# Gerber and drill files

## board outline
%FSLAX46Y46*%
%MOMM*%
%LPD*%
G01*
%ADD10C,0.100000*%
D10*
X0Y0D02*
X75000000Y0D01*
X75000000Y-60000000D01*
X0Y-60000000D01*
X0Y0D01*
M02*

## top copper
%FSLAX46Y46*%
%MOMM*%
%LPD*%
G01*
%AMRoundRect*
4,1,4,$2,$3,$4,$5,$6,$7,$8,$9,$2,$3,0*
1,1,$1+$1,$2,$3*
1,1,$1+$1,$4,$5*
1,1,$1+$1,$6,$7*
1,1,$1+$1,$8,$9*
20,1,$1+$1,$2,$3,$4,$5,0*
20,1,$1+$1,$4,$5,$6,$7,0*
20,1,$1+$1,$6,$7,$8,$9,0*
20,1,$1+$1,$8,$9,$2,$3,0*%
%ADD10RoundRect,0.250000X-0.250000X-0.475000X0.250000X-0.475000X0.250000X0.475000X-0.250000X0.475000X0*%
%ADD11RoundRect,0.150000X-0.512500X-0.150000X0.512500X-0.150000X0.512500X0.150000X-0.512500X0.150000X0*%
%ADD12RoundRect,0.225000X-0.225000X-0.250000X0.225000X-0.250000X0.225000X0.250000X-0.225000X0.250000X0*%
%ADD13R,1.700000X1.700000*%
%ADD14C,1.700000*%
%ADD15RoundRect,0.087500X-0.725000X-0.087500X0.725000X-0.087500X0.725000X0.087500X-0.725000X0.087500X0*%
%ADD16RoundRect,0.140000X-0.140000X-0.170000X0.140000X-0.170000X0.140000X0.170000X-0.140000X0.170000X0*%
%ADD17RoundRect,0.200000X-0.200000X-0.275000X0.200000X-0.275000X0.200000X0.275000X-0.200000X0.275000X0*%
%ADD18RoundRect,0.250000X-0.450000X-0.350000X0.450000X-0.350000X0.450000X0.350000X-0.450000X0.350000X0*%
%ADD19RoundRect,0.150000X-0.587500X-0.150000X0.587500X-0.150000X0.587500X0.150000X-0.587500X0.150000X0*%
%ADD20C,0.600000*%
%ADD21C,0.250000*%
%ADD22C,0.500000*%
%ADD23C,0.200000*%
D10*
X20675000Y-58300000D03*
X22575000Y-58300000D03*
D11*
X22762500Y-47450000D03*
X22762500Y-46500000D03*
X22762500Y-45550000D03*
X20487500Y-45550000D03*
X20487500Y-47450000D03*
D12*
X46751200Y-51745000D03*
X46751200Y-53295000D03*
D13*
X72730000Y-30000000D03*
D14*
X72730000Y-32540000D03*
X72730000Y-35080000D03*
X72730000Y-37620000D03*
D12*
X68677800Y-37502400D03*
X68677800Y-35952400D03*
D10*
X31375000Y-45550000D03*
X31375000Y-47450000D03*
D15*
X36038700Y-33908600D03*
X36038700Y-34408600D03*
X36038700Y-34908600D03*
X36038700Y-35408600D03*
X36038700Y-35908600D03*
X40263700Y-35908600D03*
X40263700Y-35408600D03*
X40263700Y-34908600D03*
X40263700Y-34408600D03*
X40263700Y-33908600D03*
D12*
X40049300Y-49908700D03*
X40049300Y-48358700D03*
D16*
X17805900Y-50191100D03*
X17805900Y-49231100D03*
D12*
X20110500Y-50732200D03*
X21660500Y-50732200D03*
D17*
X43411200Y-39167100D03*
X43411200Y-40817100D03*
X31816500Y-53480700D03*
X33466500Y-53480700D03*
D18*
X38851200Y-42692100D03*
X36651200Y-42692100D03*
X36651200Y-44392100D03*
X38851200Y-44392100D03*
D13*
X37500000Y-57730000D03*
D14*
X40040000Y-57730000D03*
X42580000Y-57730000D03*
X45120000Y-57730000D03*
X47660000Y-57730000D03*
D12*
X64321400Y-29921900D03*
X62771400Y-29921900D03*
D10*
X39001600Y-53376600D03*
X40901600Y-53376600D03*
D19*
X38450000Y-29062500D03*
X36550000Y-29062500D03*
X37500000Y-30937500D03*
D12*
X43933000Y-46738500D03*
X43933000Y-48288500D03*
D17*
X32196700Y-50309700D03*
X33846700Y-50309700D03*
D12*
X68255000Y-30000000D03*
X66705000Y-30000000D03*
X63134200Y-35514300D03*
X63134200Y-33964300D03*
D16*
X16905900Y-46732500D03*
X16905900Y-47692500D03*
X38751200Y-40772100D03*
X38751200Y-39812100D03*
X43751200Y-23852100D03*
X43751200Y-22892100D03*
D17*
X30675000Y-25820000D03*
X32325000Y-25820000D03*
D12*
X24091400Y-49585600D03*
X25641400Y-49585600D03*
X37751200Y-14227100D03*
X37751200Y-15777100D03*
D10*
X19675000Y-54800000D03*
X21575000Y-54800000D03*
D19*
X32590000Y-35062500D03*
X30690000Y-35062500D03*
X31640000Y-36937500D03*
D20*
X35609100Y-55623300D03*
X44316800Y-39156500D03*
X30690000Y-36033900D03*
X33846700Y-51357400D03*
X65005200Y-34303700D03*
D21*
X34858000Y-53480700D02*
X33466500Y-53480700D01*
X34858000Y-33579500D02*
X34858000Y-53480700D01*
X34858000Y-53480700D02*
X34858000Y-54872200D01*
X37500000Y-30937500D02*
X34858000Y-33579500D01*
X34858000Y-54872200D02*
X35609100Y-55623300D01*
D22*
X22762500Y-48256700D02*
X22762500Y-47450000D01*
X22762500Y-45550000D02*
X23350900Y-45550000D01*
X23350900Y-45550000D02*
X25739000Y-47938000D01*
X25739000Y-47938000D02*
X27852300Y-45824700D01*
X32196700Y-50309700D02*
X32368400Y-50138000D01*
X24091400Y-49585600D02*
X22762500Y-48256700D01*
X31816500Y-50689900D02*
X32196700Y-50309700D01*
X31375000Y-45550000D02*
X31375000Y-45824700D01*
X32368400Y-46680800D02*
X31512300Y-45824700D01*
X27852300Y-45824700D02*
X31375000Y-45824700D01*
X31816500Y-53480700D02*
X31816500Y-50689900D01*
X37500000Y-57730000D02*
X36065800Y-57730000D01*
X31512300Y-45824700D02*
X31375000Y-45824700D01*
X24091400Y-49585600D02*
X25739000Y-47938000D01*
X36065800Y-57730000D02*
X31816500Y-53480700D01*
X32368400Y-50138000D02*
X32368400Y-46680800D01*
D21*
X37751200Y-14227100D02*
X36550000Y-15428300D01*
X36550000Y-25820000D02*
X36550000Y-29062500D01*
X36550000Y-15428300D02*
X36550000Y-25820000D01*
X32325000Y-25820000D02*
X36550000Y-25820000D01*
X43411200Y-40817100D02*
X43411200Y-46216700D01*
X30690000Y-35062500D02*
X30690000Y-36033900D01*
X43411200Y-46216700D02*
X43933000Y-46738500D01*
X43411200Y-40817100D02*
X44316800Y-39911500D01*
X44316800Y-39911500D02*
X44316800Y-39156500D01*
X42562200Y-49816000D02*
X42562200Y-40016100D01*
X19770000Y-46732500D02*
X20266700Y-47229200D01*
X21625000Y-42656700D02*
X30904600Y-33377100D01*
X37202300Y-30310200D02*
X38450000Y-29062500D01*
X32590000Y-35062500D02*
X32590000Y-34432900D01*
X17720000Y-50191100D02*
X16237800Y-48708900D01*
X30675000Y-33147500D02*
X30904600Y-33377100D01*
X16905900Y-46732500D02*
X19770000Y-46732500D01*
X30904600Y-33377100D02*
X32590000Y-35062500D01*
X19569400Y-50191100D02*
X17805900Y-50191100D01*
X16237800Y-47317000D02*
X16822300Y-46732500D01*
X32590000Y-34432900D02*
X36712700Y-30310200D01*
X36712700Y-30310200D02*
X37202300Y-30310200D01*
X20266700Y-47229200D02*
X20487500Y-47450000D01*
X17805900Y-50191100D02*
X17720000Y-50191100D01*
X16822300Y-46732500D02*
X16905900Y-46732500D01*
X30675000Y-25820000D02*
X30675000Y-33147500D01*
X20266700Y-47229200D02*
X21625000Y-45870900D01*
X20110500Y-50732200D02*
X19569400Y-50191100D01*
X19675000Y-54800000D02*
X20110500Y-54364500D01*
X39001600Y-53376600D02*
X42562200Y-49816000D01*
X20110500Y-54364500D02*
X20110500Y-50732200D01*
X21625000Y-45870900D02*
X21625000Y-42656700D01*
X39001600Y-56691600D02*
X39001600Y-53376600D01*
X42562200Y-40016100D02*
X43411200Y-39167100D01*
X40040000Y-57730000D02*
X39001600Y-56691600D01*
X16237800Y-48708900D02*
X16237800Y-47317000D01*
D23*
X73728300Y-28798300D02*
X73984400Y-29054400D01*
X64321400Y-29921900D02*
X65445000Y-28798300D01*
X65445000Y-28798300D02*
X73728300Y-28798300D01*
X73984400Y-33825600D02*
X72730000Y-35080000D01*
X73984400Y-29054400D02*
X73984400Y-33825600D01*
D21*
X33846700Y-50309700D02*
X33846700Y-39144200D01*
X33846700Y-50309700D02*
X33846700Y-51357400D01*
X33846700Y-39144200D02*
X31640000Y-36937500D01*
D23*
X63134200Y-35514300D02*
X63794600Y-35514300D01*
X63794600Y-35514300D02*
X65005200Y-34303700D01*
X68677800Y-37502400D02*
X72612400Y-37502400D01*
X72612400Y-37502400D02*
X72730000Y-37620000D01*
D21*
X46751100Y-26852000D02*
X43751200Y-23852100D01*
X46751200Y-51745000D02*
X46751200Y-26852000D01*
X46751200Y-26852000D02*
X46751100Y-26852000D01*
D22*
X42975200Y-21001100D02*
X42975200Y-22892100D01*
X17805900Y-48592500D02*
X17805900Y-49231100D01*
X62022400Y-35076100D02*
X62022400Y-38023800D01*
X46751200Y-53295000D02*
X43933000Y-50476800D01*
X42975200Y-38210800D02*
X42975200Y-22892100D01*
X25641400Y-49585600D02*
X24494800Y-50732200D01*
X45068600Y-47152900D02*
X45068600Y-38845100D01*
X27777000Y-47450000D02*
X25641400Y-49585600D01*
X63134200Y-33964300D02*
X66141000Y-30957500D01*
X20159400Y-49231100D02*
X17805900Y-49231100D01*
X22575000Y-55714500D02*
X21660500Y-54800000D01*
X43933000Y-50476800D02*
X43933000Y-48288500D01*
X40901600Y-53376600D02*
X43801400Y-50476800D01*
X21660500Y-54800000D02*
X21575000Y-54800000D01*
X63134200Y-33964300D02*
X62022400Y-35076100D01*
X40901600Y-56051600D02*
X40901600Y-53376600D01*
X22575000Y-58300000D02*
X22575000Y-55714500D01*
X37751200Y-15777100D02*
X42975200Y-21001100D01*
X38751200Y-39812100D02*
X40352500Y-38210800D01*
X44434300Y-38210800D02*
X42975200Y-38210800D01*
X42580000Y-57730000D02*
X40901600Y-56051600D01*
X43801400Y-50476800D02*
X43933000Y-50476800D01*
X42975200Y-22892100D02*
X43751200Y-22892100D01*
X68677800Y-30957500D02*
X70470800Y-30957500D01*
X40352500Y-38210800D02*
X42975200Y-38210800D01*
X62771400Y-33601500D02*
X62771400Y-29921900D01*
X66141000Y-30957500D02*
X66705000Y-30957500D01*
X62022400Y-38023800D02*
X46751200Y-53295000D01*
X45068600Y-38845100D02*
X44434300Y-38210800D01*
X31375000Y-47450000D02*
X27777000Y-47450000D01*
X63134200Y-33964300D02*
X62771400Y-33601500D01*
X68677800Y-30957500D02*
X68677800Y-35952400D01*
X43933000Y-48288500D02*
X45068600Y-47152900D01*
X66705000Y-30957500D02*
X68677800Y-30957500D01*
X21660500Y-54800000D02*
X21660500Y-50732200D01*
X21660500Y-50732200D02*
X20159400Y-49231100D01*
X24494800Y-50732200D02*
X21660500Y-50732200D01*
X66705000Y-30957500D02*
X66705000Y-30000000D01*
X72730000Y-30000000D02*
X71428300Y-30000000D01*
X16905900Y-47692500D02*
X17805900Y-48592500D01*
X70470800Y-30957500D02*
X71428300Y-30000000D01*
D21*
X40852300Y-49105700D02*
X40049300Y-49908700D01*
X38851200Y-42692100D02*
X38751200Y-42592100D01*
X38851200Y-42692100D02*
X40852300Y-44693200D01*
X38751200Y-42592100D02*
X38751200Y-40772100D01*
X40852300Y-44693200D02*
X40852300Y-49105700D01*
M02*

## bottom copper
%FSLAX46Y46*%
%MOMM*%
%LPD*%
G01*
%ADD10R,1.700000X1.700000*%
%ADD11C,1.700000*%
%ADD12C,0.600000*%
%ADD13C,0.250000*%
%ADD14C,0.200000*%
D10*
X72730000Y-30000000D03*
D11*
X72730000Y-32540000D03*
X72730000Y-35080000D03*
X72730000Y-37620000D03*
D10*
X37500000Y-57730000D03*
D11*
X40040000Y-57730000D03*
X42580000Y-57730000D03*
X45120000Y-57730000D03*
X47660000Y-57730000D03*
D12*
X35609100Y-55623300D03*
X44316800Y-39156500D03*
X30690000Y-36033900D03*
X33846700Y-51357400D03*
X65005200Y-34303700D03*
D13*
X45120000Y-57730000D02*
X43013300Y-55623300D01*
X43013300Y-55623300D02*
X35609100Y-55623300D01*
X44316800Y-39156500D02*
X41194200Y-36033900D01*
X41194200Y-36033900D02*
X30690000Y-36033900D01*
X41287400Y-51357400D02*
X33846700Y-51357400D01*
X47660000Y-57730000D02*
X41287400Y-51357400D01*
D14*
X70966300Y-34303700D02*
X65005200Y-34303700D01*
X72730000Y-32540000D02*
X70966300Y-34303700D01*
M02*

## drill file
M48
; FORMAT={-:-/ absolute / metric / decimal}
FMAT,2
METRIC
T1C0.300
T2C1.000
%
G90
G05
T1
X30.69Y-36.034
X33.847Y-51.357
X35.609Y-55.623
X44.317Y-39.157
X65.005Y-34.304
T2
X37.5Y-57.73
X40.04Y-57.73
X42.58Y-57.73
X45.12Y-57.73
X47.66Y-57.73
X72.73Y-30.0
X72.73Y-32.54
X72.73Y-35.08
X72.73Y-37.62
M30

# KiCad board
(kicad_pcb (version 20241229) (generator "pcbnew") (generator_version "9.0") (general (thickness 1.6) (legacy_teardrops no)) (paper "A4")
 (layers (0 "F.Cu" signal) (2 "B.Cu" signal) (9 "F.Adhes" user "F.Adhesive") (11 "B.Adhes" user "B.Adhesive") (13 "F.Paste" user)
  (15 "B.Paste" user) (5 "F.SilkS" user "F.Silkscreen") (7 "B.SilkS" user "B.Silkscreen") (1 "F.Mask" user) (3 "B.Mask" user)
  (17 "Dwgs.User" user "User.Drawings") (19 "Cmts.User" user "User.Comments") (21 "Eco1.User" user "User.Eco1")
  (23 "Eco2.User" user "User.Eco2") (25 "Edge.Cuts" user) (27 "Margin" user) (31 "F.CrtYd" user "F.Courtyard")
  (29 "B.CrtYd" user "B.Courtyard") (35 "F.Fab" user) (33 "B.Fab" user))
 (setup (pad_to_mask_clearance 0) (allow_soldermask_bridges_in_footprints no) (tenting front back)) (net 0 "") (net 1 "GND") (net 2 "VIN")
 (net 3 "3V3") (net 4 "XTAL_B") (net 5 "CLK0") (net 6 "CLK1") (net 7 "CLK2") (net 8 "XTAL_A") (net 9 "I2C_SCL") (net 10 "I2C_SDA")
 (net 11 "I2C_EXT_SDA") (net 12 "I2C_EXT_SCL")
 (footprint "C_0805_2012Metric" (layer "F.Cu") (at 21.625 58.3)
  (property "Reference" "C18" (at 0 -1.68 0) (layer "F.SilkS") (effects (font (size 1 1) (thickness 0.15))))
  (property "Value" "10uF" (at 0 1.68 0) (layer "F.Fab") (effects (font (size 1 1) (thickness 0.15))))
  (pad "1" smd roundrect (at -0.95 0) (size 1 1.45) (layers "F.Cu" "F.Mask" "F.Paste") (roundrect_rratio 0.25))
  (pad "2" smd roundrect (at 0.95 0) (size 1 1.45) (layers "F.Cu" "F.Mask" "F.Paste") (roundrect_rratio 0.25) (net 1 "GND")))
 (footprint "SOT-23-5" (layer "F.Cu") (at 21.625 46.5 180)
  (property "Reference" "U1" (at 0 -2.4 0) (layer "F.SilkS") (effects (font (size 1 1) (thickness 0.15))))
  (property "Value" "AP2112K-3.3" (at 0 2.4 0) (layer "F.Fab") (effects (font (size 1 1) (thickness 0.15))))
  (pad "1" smd roundrect (at -1.1375 -0.95) (size 1.325 0.6) (layers "F.Cu" "F.Mask" "F.Paste") (roundrect_rratio 0.25) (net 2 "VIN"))
  (pad "2" smd roundrect (at -1.1375 0) (size 1.325 0.6) (layers "F.Cu" "F.Mask" "F.Paste") (roundrect_rratio 0.25) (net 1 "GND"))
  (pad "3" smd roundrect (at -1.1375 0.95) (size 1.325 0.6) (layers "F.Cu" "F.Mask" "F.Paste") (roundrect_rratio 0.25) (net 2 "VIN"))
  (pad "4" smd roundrect (at 1.1375 0.95) (size 1.325 0.6) (layers "F.Cu" "F.Mask" "F.Paste") (roundrect_rratio 0.25))
  (pad "5" smd roundrect (at 1.1375 -0.95) (size 1.325 0.6) (layers "F.Cu" "F.Mask" "F.Paste") (roundrect_rratio 0.25) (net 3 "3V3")))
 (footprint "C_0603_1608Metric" (layer "F.Cu") (at 46.7512 52.52 -90)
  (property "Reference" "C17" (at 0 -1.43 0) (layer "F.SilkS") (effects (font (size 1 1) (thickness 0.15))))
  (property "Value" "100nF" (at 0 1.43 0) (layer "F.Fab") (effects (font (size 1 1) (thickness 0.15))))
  (pad "1" smd roundrect (at -0.775 0) (size 0.9 0.95) (layers "F.Cu" "F.Mask" "F.Paste") (roundrect_rratio 0.25) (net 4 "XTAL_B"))
  (pad "2" smd roundrect (at 0.775 0) (size 0.9 0.95) (layers "F.Cu" "F.Mask" "F.Paste") (roundrect_rratio 0.25) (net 1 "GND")))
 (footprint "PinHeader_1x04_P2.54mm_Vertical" (layer "F.Cu") (at 72.73 30)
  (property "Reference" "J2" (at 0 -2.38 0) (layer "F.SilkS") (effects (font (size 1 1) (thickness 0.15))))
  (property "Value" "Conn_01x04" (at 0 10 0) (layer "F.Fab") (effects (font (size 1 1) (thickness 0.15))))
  (pad "1" thru_hole rect (at 0 0) (size 1.7 1.7) (drill 1) (layers "*.Cu" "*.Mask") (remove_unused_layers no) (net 1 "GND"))
  (pad "2" thru_hole circle (at 0 2.54) (size 1.7 1.7) (drill 1) (layers "*.Cu" "*.Mask") (remove_unused_layers no) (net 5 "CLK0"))
  (pad "3" thru_hole circle (at 0 5.08) (size 1.7 1.7) (drill 1) (layers "*.Cu" "*.Mask") (remove_unused_layers no) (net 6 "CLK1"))
  (pad "4" thru_hole circle (at 0 7.62) (size 1.7 1.7) (drill 1) (layers "*.Cu" "*.Mask") (remove_unused_layers no) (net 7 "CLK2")))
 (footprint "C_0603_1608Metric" (layer "F.Cu") (at 68.6778 36.7274 90)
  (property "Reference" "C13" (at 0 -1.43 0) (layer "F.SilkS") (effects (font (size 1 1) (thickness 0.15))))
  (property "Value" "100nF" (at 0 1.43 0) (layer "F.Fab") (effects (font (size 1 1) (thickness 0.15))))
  (pad "1" smd roundrect (at -0.775 0) (size 0.9 0.95) (layers "F.Cu" "F.Mask" "F.Paste") (roundrect_rratio 0.25) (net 7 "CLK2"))
  (pad "2" smd roundrect (at 0.775 0) (size 0.9 0.95) (layers "F.Cu" "F.Mask" "F.Paste") (roundrect_rratio 0.25) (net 1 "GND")))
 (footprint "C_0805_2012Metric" (layer "F.Cu") (at 31.375 46.5 -90)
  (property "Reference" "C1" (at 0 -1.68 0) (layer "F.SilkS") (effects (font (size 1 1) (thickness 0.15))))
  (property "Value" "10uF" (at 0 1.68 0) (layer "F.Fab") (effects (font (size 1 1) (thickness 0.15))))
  (pad "1" smd roundrect (at -0.95 0) (size 1 1.45) (layers "F.Cu" "F.Mask" "F.Paste") (roundrect_rratio 0.25) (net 2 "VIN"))
  (pad "2" smd roundrect (at 0.95 0) (size 1 1.45) (layers "F.Cu" "F.Mask" "F.Paste") (roundrect_rratio 0.25) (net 1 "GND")))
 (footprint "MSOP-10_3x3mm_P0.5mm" (layer "F.Cu") (at 38.1512 34.9086)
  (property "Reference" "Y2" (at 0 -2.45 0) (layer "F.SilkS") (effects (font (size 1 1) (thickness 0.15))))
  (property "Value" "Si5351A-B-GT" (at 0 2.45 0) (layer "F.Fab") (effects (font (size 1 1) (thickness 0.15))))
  (pad "1" smd roundrect (at -2.1125 -1) (size 1.625 0.35) (layers "F.Cu" "F.Mask" "F.Paste") (roundrect_rratio 0.25) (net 3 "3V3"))
  (pad "2" smd roundrect (at -2.1125 -0.5) (size 1.625 0.35) (layers "F.Cu" "F.Mask" "F.Paste") (roundrect_rratio 0.25) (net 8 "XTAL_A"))
  (pad "3" smd roundrect (at -2.1125 0) (size 1.625 0.35) (layers "F.Cu" "F.Mask" "F.Paste") (roundrect_rratio 0.25) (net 4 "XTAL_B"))
  (pad "4" smd roundrect (at -2.1125 0.5) (size 1.625 0.35) (layers "F.Cu" "F.Mask" "F.Paste") (roundrect_rratio 0.25) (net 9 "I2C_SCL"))
  (pad "5" smd roundrect (at -2.1125 1) (size 1.625 0.35) (layers "F.Cu" "F.Mask" "F.Paste") (roundrect_rratio 0.25) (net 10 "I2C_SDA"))
  (pad "6" smd roundrect (at 2.1125 1) (size 1.625 0.35) (layers "F.Cu" "F.Mask" "F.Paste") (roundrect_rratio 0.25) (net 7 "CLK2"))
  (pad "7" smd roundrect (at 2.1125 0.5) (size 1.625 0.35) (layers "F.Cu" "F.Mask" "F.Paste") (roundrect_rratio 0.25) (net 3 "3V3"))
  (pad "8" smd roundrect (at 2.1125 0) (size 1.625 0.35) (layers "F.Cu" "F.Mask" "F.Paste") (roundrect_rratio 0.25) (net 1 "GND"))
  (pad "9" smd roundrect (at 2.1125 -0.5) (size 1.625 0.35) (layers "F.Cu" "F.Mask" "F.Paste") (roundrect_rratio 0.25) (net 6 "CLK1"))
  (pad "10" smd roundrect (at 2.1125 -1) (size 1.625 0.35) (layers "F.Cu" "F.Mask" "F.Paste") (roundrect_rratio 0.25) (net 5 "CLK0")))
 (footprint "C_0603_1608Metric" (layer "F.Cu") (at 40.0493 49.1337 90)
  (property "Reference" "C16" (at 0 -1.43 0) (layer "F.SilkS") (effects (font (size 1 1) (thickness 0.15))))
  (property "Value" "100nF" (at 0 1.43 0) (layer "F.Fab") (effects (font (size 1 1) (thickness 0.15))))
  (pad "1" smd roundrect (at -0.775 0) (size 0.9 0.95) (layers "F.Cu" "F.Mask" "F.Paste") (roundrect_rratio 0.25) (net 8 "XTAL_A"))
  (pad "2" smd roundrect (at 0.775 0) (size 0.9 0.95) (layers "F.Cu" "F.Mask" "F.Paste") (roundrect_rratio 0.25) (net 1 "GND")))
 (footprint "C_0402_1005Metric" (layer "F.Cu") (at 17.8059 49.7111 90)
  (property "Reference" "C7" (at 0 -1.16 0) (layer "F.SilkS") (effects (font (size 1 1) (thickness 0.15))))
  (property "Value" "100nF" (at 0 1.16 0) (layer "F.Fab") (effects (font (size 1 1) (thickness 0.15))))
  (pad "1" smd roundrect (at -0.48 0) (size 0.56 0.62) (layers "F.Cu" "F.Mask" "F.Paste") (roundrect_rratio 0.25) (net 3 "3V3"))
  (pad "2" smd roundrect (at 0.48 0) (size 0.56 0.62) (layers "F.Cu" "F.Mask" "F.Paste") (roundrect_rratio 0.25) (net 1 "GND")))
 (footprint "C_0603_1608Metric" (layer "F.Cu") (at 20.8855 50.7322)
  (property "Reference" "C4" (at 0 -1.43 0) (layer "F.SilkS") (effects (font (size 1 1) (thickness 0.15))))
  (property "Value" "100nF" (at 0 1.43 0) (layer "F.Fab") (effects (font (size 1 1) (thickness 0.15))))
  (pad "1" smd roundrect (at -0.775 0) (size 0.9 0.95) (layers "F.Cu" "F.Mask" "F.Paste") (roundrect_rratio 0.25) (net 3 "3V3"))
  (pad "2" smd roundrect (at 0.775 0) (size 0.9 0.95) (layers "F.Cu" "F.Mask" "F.Paste") (roundrect_rratio 0.25) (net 1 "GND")))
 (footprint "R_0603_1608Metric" (layer "F.Cu") (at 43.4112 39.9921 -90)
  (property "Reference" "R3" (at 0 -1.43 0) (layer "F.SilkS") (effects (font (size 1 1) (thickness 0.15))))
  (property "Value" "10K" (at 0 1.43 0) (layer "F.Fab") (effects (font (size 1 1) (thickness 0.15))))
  (pad "1" smd roundrect (at -0.825 0) (size 0.8 0.95) (layers "F.Cu" "F.Mask" "F.Paste") (roundrect_rratio 0.25) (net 3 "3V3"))
  (pad "2" smd roundrect (at 0.825 0) (size 0.8 0.95) (layers "F.Cu" "F.Mask" "F.Paste") (roundrect_rratio 0.25) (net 9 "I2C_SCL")))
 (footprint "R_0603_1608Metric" (layer "F.Cu") (at 32.6415 53.4807)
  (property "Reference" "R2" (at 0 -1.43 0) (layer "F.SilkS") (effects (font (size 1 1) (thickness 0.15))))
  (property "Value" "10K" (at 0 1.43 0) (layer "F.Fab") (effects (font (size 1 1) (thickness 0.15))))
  (pad "1" smd roundrect (at -0.825 0) (size 0.8 0.95) (layers "F.Cu" "F.Mask" "F.Paste") (roundrect_rratio 0.25) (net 2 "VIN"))
  (pad "2" smd roundrect (at 0.825 0) (size 0.8 0.95) (layers "F.Cu" "F.Mask" "F.Paste") (roundrect_rratio 0.25) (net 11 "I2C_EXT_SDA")))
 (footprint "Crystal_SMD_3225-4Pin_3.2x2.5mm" (layer "F.Cu") (at 37.7512 43.5421 180)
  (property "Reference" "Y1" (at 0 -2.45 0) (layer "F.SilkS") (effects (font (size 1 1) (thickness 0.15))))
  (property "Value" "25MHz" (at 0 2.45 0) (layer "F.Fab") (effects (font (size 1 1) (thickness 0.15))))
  (pad "1" smd roundrect (at -1.1 0.85) (size 1.4 1.2) (layers "F.Cu" "F.Mask" "F.Paste") (roundrect_rratio 0.208333) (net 8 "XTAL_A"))
  (pad "2" smd roundrect (at 1.1 0.85) (size 1.4 1.2) (layers "F.Cu" "F.Mask" "F.Paste") (roundrect_rratio 0.208333) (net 4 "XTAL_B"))
  (pad "3" smd roundrect (at 1.1 -0.85) (size 1.4 1.2) (layers "F.Cu" "F.Mask" "F.Paste") (roundrect_rratio 0.208333))
  (pad "4" smd roundrect (at -1.1 -0.85) (size 1.4 1.2) (layers "F.Cu" "F.Mask" "F.Paste") (roundrect_rratio 0.208333)))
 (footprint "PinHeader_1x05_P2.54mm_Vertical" (layer "F.Cu") (at 37.5 57.73 90)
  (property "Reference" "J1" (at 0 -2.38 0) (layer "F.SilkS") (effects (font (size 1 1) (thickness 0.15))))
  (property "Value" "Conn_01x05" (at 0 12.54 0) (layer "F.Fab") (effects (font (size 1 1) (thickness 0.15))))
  (pad "1" thru_hole rect (at 0 0) (size 1.7 1.7) (drill 1) (layers "*.Cu" "*.Mask") (remove_unused_layers no) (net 2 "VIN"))
  (pad "2" thru_hole circle (at 0 2.54) (size 1.7 1.7) (drill 1) (layers "*.Cu" "*.Mask") (remove_unused_layers no) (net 3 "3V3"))
  (pad "3" thru_hole circle (at 0 5.08) (size 1.7 1.7) (drill 1) (layers "*.Cu" "*.Mask") (remove_unused_layers no) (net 1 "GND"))
  (pad "4" thru_hole circle (at 0 7.62) (size 1.7 1.7) (drill 1) (layers "*.Cu" "*.Mask") (remove_unused_layers no) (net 11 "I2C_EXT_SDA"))
  (pad "5" thru_hole circle (at 0 10.16) (size 1.7 1.7) (drill 1) (layers "*.Cu" "*.Mask") (remove_unused_layers no) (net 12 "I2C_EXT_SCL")))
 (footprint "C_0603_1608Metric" (layer "F.Cu") (at 63.5464 29.9219 180)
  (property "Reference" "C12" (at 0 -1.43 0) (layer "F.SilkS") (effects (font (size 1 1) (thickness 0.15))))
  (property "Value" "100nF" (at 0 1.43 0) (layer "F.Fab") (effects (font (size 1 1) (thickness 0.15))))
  (pad "1" smd roundrect (at -0.775 0) (size 0.9 0.95) (layers "F.Cu" "F.Mask" "F.Paste") (roundrect_rratio 0.25) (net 6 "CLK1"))
  (pad "2" smd roundrect (at 0.775 0) (size 0.9 0.95) (layers "F.Cu" "F.Mask" "F.Paste") (roundrect_rratio 0.25) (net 1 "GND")))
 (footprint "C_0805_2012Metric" (layer "F.Cu") (at 39.9516 53.3766)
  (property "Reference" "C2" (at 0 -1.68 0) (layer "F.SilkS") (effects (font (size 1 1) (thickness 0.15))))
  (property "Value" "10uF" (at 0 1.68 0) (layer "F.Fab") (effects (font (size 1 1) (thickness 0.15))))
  (pad "1" smd roundrect (at -0.95 0) (size 1 1.45) (layers "F.Cu" "F.Mask" "F.Paste") (roundrect_rratio 0.25) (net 3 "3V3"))
  (pad "2" smd roundrect (at 0.95 0) (size 1 1.45) (layers "F.Cu" "F.Mask" "F.Paste") (roundrect_rratio 0.25) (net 1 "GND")))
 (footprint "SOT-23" (layer "F.Cu") (at 37.5 30 -90)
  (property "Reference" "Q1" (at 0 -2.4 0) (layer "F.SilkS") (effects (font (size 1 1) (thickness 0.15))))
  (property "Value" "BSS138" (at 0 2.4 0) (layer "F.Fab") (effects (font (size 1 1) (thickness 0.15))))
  (pad "1" smd roundrect (at -0.9375 -0.95) (size 1.475 0.6) (layers "F.Cu" "F.Mask" "F.Paste") (roundrect_rratio 0.25) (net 3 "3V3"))
  (pad "2" smd roundrect (at -0.9375 0.95) (size 1.475 0.6) (layers "F.Cu" "F.Mask" "F.Paste") (roundrect_rratio 0.25) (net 10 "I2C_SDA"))
  (pad "3" smd roundrect (at 0.9375 0) (size 1.475 0.6) (layers "F.Cu" "F.Mask" "F.Paste") (roundrect_rratio 0.25) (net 11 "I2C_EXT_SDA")))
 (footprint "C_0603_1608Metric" (layer "F.Cu") (at 43.933 47.5135 -90)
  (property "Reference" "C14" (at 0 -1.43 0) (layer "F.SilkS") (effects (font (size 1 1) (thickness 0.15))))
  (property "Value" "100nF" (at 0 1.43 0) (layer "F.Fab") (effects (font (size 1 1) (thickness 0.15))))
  (pad "1" smd roundrect (at -0.775 0) (size 0.9 0.95) (layers "F.Cu" "F.Mask" "F.Paste") (roundrect_rratio 0.25) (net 9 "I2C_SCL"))
  (pad "2" smd roundrect (at 0.775 0) (size 0.9 0.95) (layers "F.Cu" "F.Mask" "F.Paste") (roundrect_rratio 0.25) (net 1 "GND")))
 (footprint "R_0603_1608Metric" (layer "F.Cu") (at 33.0217 50.3097)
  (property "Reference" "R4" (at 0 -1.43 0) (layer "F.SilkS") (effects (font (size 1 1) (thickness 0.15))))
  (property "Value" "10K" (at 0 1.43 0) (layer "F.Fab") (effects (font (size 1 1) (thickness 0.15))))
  (pad "1" smd roundrect (at -0.825 0) (size 0.8 0.95) (layers "F.Cu" "F.Mask" "F.Paste") (roundrect_rratio 0.25) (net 2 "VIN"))
  (pad "2" smd roundrect (at 0.825 0) (size 0.8 0.95) (layers "F.Cu" "F.Mask" "F.Paste") (roundrect_rratio 0.25) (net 12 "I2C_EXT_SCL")))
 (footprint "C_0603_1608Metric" (layer "F.Cu") (at 67.48 30 180)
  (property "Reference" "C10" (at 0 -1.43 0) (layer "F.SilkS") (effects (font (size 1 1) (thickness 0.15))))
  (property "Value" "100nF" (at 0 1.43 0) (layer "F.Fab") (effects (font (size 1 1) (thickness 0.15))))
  (pad "1" smd roundrect (at -0.775 0) (size 0.9 0.95) (layers "F.Cu" "F.Mask" "F.Paste") (roundrect_rratio 0.25))
  (pad "2" smd roundrect (at 0.775 0) (size 0.9 0.95) (layers "F.Cu" "F.Mask" "F.Paste") (roundrect_rratio 0.25) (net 1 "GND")))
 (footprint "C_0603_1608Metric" (layer "F.Cu") (at 63.1342 34.7393 90)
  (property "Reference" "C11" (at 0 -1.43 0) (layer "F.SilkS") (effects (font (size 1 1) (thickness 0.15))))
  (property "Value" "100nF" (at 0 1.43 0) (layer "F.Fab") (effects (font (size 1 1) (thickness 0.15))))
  (pad "1" smd roundrect (at -0.775 0) (size 0.9 0.95) (layers "F.Cu" "F.Mask" "F.Paste") (roundrect_rratio 0.25) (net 5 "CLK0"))
  (pad "2" smd roundrect (at 0.775 0) (size 0.9 0.95) (layers "F.Cu" "F.Mask" "F.Paste") (roundrect_rratio 0.25) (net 1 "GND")))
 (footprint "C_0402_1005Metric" (layer "F.Cu") (at 16.9059 47.2125 -90)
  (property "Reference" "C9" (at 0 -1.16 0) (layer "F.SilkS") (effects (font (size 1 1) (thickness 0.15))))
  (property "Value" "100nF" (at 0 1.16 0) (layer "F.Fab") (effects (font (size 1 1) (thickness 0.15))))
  (pad "1" smd roundrect (at -0.48 0) (size 0.56 0.62) (layers "F.Cu" "F.Mask" "F.Paste") (roundrect_rratio 0.25) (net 3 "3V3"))
  (pad "2" smd roundrect (at 0.48 0) (size 0.56 0.62) (layers "F.Cu" "F.Mask" "F.Paste") (roundrect_rratio 0.25) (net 1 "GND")))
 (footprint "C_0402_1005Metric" (layer "F.Cu") (at 38.7512 40.2921 90)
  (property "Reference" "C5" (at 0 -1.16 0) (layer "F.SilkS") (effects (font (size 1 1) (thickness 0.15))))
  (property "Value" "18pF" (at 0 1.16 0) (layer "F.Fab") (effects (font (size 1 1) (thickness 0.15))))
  (pad "1" smd roundrect (at -0.48 0) (size 0.56 0.62) (layers "F.Cu" "F.Mask" "F.Paste") (roundrect_rratio 0.25) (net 8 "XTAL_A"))
  (pad "2" smd roundrect (at 0.48 0) (size 0.56 0.62) (layers "F.Cu" "F.Mask" "F.Paste") (roundrect_rratio 0.25) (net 1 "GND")))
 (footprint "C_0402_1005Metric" (layer "F.Cu") (at 43.7512 23.3721 90)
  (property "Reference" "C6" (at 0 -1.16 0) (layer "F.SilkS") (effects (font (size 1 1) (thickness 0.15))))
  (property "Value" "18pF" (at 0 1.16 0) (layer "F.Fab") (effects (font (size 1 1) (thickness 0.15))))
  (pad "1" smd roundrect (at -0.48 0) (size 0.56 0.62) (layers "F.Cu" "F.Mask" "F.Paste") (roundrect_rratio 0.25) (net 4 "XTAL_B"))
  (pad "2" smd roundrect (at 0.48 0) (size 0.56 0.62) (layers "F.Cu" "F.Mask" "F.Paste") (roundrect_rratio 0.25) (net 1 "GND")))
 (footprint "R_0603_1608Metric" (layer "F.Cu") (at 31.5 25.82)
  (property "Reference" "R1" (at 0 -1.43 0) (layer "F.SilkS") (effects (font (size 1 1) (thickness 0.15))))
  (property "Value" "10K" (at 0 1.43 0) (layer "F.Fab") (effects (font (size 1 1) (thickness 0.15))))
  (pad "1" smd roundrect (at -0.825 0) (size 0.8 0.95) (layers "F.Cu" "F.Mask" "F.Paste") (roundrect_rratio 0.25) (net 3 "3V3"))
  (pad "2" smd roundrect (at 0.825 0) (size 0.8 0.95) (layers "F.Cu" "F.Mask" "F.Paste") (roundrect_rratio 0.25) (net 10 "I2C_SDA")))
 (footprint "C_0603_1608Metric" (layer "F.Cu") (at 24.8664 49.5856)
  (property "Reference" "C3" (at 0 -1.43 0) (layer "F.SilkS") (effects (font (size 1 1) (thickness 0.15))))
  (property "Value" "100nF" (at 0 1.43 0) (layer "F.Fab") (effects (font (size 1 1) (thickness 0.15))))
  (pad "1" smd roundrect (at -0.775 0) (size 0.9 0.95) (layers "F.Cu" "F.Mask" "F.Paste") (roundrect_rratio 0.25) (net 2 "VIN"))
  (pad "2" smd roundrect (at 0.775 0) (size 0.9 0.95) (layers "F.Cu" "F.Mask" "F.Paste") (roundrect_rratio 0.25) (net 1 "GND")))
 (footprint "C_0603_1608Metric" (layer "F.Cu") (at 37.7512 15.0021 -90)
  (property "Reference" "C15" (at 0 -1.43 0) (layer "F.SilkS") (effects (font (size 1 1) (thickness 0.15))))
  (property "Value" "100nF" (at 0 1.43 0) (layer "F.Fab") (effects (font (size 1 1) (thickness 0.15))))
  (pad "1" smd roundrect (at -0.775 0) (size 0.9 0.95) (layers "F.Cu" "F.Mask" "F.Paste") (roundrect_rratio 0.25) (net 10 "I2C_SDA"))
  (pad "2" smd roundrect (at 0.775 0) (size 0.9 0.95) (layers "F.Cu" "F.Mask" "F.Paste") (roundrect_rratio 0.25) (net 1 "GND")))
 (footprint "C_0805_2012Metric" (layer "F.Cu") (at 20.625 54.8)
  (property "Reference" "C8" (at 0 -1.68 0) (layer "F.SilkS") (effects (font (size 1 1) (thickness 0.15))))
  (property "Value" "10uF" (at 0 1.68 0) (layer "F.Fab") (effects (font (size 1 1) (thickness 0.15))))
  (pad "1" smd roundrect (at -0.95 0) (size 1 1.45) (layers "F.Cu" "F.Mask" "F.Paste") (roundrect_rratio 0.25) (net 3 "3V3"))
  (pad "2" smd roundrect (at 0.95 0) (size 1 1.45) (layers "F.Cu" "F.Mask" "F.Paste") (roundrect_rratio 0.25) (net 1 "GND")))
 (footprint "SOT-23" (layer "F.Cu") (at 31.64 36 -90)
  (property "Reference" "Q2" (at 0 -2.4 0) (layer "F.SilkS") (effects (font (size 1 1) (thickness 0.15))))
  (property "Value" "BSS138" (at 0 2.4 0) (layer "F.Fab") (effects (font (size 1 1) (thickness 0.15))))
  (pad "1" smd roundrect (at -0.9375 -0.95) (size 1.475 0.6) (layers "F.Cu" "F.Mask" "F.Paste") (roundrect_rratio 0.25) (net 3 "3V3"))
  (pad "2" smd roundrect (at -0.9375 0.95) (size 1.475 0.6) (layers "F.Cu" "F.Mask" "F.Paste") (roundrect_rratio 0.25) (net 9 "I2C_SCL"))
  (pad "3" smd roundrect (at 0.9375 0) (size 1.475 0.6) (layers "F.Cu" "F.Mask" "F.Paste") (roundrect_rratio 0.25) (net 12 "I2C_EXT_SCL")))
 (gr_rect (start 0 0) (end 75 60) (stroke (width 0.1) (type solid)) (fill no) (layer "Edge.Cuts"))
 (segment (start 34.858 53.4807) (end 33.4665 53.4807) (width 0.25) (layer "F.Cu") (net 11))
 (segment (start 34.858 33.5795) (end 34.858 53.4807) (width 0.25) (layer "F.Cu") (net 11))
 (segment (start 34.858 53.4807) (end 34.858 54.8722) (width 0.25) (layer "F.Cu") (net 11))
 (segment (start 37.5 30.9375) (end 34.858 33.5795) (width 0.25) (layer "F.Cu") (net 11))
 (segment (start 34.858 54.8722) (end 35.6091 55.6233) (width 0.25) (layer "F.Cu") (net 11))
 (via (at 35.6091 55.6233) (size 0.6) (drill 0.3) (layers "F.Cu" "B.Cu") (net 11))
 (segment (start 45.12 57.73) (end 43.0133 55.6233) (width 0.25) (layer "B.Cu") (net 11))
 (segment (start 43.0133 55.6233) (end 35.6091 55.6233) (width 0.25) (layer "B.Cu") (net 11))
 (segment (start 22.7625 48.2567) (end 22.7625 47.45) (width 0.5) (layer "F.Cu") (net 2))
 (segment (start 22.7625 45.55) (end 23.3509 45.55) (width 0.5) (layer "F.Cu") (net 2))
 (segment (start 23.3509 45.55) (end 25.739 47.938) (width 0.5) (layer "F.Cu") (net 2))
 (segment (start 25.739 47.938) (end 27.8523 45.8247) (width 0.5) (layer "F.Cu") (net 2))
 (segment (start 32.1967 50.3097) (end 32.3684 50.138) (width 0.5) (layer "F.Cu") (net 2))
 (segment (start 24.0914 49.5856) (end 22.7625 48.2567) (width 0.5) (layer "F.Cu") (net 2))
 (segment (start 31.8165 50.6899) (end 32.1967 50.3097) (width 0.5) (layer "F.Cu") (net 2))
 (segment (start 31.375 45.55) (end 31.375 45.8247) (width 0.5) (layer "F.Cu") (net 2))
 (segment (start 32.3684 46.6808) (end 31.5123 45.8247) (width 0.5) (layer "F.Cu") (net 2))
 (segment (start 27.8523 45.8247) (end 31.375 45.8247) (width 0.5) (layer "F.Cu") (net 2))
 (segment (start 31.8165 53.4807) (end 31.8165 50.6899) (width 0.5) (layer "F.Cu") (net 2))
 (segment (start 37.5 57.73) (end 36.0658 57.73) (width 0.5) (layer "F.Cu") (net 2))
 (segment (start 31.5123 45.8247) (end 31.375 45.8247) (width 0.5) (layer "F.Cu") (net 2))
 (segment (start 24.0914 49.5856) (end 25.739 47.938) (width 0.5) (layer "F.Cu") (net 2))
 (segment (start 36.0658 57.73) (end 31.8165 53.4807) (width 0.5) (layer "F.Cu") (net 2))
 (segment (start 32.3684 50.138) (end 32.3684 46.6808) (width 0.5) (layer "F.Cu") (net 2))
 (segment (start 37.7512 14.2271) (end 36.55 15.4283) (width 0.25) (layer "F.Cu") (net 10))
 (segment (start 36.55 25.82) (end 36.55 29.0625) (width 0.25) (layer "F.Cu") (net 10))
 (segment (start 36.55 15.4283) (end 36.55 25.82) (width 0.25) (layer "F.Cu") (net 10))
 (segment (start 32.325 25.82) (end 36.55 25.82) (width 0.25) (layer "F.Cu") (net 10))
 (segment (start 43.4112 40.8171) (end 43.4112 46.2167) (width 0.25) (layer "F.Cu") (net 9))
 (segment (start 30.69 35.0625) (end 30.69 36.0339) (width 0.25) (layer "F.Cu") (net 9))
 (segment (start 43.4112 46.2167) (end 43.933 46.7385) (width 0.25) (layer "F.Cu") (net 9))
 (segment (start 43.4112 40.8171) (end 44.3168 39.9115) (width 0.25) (layer "F.Cu") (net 9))
 (segment (start 44.3168 39.9115) (end 44.3168 39.1565) (width 0.25) (layer "F.Cu") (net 9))
 (via (at 44.3168 39.1565) (size 0.6) (drill 0.3) (layers "F.Cu" "B.Cu") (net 9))
 (via (at 30.69 36.0339) (size 0.6) (drill 0.3) (layers "F.Cu" "B.Cu") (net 9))
 (segment (start 44.3168 39.1565) (end 41.1942 36.0339) (width 0.25) (layer "B.Cu") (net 9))
 (segment (start 41.1942 36.0339) (end 30.69 36.0339) (width 0.25) (layer "B.Cu") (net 9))
 (segment (start 42.5622 49.816) (end 42.5622 40.0161) (width 0.25) (layer "F.Cu") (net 3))
 (segment (start 19.77 46.7325) (end 20.2667 47.2292) (width 0.25) (layer "F.Cu") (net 3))
 (segment (start 21.625 42.6567) (end 30.9046 33.3771) (width 0.25) (layer "F.Cu") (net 3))
 (segment (start 37.2023 30.3102) (end 38.45 29.0625) (width 0.25) (layer "F.Cu") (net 3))
 (segment (start 32.59 35.0625) (end 32.59 34.4329) (width 0.25) (layer "F.Cu") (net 3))
 (segment (start 17.72 50.1911) (end 16.2378 48.7089) (width 0.25) (layer "F.Cu") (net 3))
 (segment (start 30.675 33.1475) (end 30.9046 33.3771) (width 0.25) (layer "F.Cu") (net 3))
 (segment (start 16.9059 46.7325) (end 19.77 46.7325) (width 0.25) (layer "F.Cu") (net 3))
 (segment (start 30.9046 33.3771) (end 32.59 35.0625) (width 0.25) (layer "F.Cu") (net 3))
 (segment (start 19.5694 50.1911) (end 17.8059 50.1911) (width 0.25) (layer "F.Cu") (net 3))
 (segment (start 16.2378 47.317) (end 16.8223 46.7325) (width 0.25) (layer "F.Cu") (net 3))
 (segment (start 32.59 34.4329) (end 36.7127 30.3102) (width 0.25) (layer "F.Cu") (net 3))
 (segment (start 36.7127 30.3102) (end 37.2023 30.3102) (width 0.25) (layer "F.Cu") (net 3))
 (segment (start 20.2667 47.2292) (end 20.4875 47.45) (width 0.25) (layer "F.Cu") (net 3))
 (segment (start 17.8059 50.1911) (end 17.72 50.1911) (width 0.25) (layer "F.Cu") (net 3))
 (segment (start 16.8223 46.7325) (end 16.9059 46.7325) (width 0.25) (layer "F.Cu") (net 3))
 (segment (start 30.675 25.82) (end 30.675 33.1475) (width 0.25) (layer "F.Cu") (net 3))
 (segment (start 20.2667 47.2292) (end 21.625 45.8709) (width 0.25) (layer "F.Cu") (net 3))
 (segment (start 20.1105 50.7322) (end 19.5694 50.1911) (width 0.25) (layer "F.Cu") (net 3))
 (segment (start 19.675 54.8) (end 20.1105 54.3645) (width 0.25) (layer "F.Cu") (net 3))
 (segment (start 39.0016 53.3766) (end 42.5622 49.816) (width 0.25) (layer "F.Cu") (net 3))
 (segment (start 20.1105 54.3645) (end 20.1105 50.7322) (width 0.25) (layer "F.Cu") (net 3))
 (segment (start 21.625 45.8709) (end 21.625 42.6567) (width 0.25) (layer "F.Cu") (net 3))
 (segment (start 39.0016 56.6916) (end 39.0016 53.3766) (width 0.25) (layer "F.Cu") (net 3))
 (segment (start 42.5622 40.0161) (end 43.4112 39.1671) (width 0.25) (layer "F.Cu") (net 3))
 (segment (start 40.04 57.73) (end 39.0016 56.6916) (width 0.25) (layer "F.Cu") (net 3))
 (segment (start 16.2378 48.7089) (end 16.2378 47.317) (width 0.25) (layer "F.Cu") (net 3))
 (segment (start 73.7283 28.7983) (end 73.9844 29.0544) (width 0.2) (layer "F.Cu") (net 6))
 (segment (start 64.3214 29.9219) (end 65.445 28.7983) (width 0.2) (layer "F.Cu") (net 6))
 (segment (start 65.445 28.7983) (end 73.7283 28.7983) (width 0.2) (layer "F.Cu") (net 6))
 (segment (start 73.9844 33.8256) (end 72.73 35.08) (width 0.2) (layer "F.Cu") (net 6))
 (segment (start 73.9844 29.0544) (end 73.9844 33.8256) (width 0.2) (layer "F.Cu") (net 6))
 (segment (start 33.8467 50.3097) (end 33.8467 39.1442) (width 0.25) (layer "F.Cu") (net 12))
 (segment (start 33.8467 50.3097) (end 33.8467 51.3574) (width 0.25) (layer "F.Cu") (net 12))
 (segment (start 33.8467 39.1442) (end 31.64 36.9375) (width 0.25) (layer "F.Cu") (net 12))
 (via (at 33.8467 51.3574) (size 0.6) (drill 0.3) (layers "F.Cu" "B.Cu") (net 12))
 (segment (start 41.2874 51.3574) (end 33.8467 51.3574) (width 0.25) (layer "B.Cu") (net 12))
 (segment (start 47.66 57.73) (end 41.2874 51.3574) (width 0.25) (layer "B.Cu") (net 12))
 (segment (start 63.1342 35.5143) (end 63.7946 35.5143) (width 0.2) (layer "F.Cu") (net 5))
 (segment (start 63.7946 35.5143) (end 65.0052 34.3037) (width 0.2) (layer "F.Cu") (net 5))
 (via (at 65.0052 34.3037) (size 0.6) (drill 0.3) (layers "F.Cu" "B.Cu") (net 5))
 (segment (start 70.9663 34.3037) (end 65.0052 34.3037) (width 0.2) (layer "B.Cu") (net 5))
 (segment (start 72.73 32.54) (end 70.9663 34.3037) (width 0.2) (layer "B.Cu") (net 5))
 (segment (start 68.6778 37.5024) (end 72.6124 37.5024) (width 0.2) (layer "F.Cu") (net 7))
 (segment (start 72.6124 37.5024) (end 72.73 37.62) (width 0.2) (layer "F.Cu") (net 7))
 (segment (start 46.7511 26.852) (end 43.7512 23.8521) (width 0.25) (layer "F.Cu") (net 4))
 (segment (start 46.7512 51.745) (end 46.7512 26.852) (width 0.25) (layer "F.Cu") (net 4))
 (segment (start 46.7512 26.852) (end 46.7511 26.852) (width 0.25) (layer "F.Cu") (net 4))
 (segment (start 42.9752 21.0011) (end 42.9752 22.8921) (width 0.5) (layer "F.Cu") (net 1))
 (segment (start 17.8059 48.5925) (end 17.8059 49.2311) (width 0.5) (layer "F.Cu") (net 1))
 (segment (start 62.0224 35.0761) (end 62.0224 38.0238) (width 0.5) (layer "F.Cu") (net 1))
 (segment (start 46.7512 53.295) (end 43.933 50.4768) (width 0.5) (layer "F.Cu") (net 1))
 (segment (start 42.9752 38.2108) (end 42.9752 22.8921) (width 0.5) (layer "F.Cu") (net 1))
 (segment (start 25.6414 49.5856) (end 24.4948 50.7322) (width 0.5) (layer "F.Cu") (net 1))
 (segment (start 45.0686 47.1529) (end 45.0686 38.8451) (width 0.5) (layer "F.Cu") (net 1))
 (segment (start 27.777 47.45) (end 25.6414 49.5856) (width 0.5) (layer "F.Cu") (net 1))
 (segment (start 63.1342 33.9643) (end 66.141 30.9575) (width 0.5) (layer "F.Cu") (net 1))
 (segment (start 20.1594 49.2311) (end 17.8059 49.2311) (width 0.5) (layer "F.Cu") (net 1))
 (segment (start 22.575 55.7145) (end 21.6605 54.8) (width 0.5) (layer "F.Cu") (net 1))
 (segment (start 43.933 50.4768) (end 43.933 48.2885) (width 0.5) (layer "F.Cu") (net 1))
 (segment (start 40.9016 53.3766) (end 43.8014 50.4768) (width 0.5) (layer "F.Cu") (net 1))
 (segment (start 21.6605 54.8) (end 21.575 54.8) (width 0.5) (layer "F.Cu") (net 1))
 (segment (start 63.1342 33.9643) (end 62.0224 35.0761) (width 0.5) (layer "F.Cu") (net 1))
 (segment (start 40.9016 56.0516) (end 40.9016 53.3766) (width 0.5) (layer "F.Cu") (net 1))
 (segment (start 22.575 58.3) (end 22.575 55.7145) (width 0.5) (layer "F.Cu") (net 1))
 (segment (start 37.7512 15.7771) (end 42.9752 21.0011) (width 0.5) (layer "F.Cu") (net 1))
 (segment (start 38.7512 39.8121) (end 40.3525 38.2108) (width 0.5) (layer "F.Cu") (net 1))
 (segment (start 44.4343 38.2108) (end 42.9752 38.2108) (width 0.5) (layer "F.Cu") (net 1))
 (segment (start 42.58 57.73) (end 40.9016 56.0516) (width 0.5) (layer "F.Cu") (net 1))
 (segment (start 43.8014 50.4768) (end 43.933 50.4768) (width 0.5) (layer "F.Cu") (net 1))
 (segment (start 42.9752 22.8921) (end 43.7512 22.8921) (width 0.5) (layer "F.Cu") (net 1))
 (segment (start 68.6778 30.9575) (end 70.4708 30.9575) (width 0.5) (layer "F.Cu") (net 1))
 (segment (start 40.3525 38.2108) (end 42.9752 38.2108) (width 0.5) (layer "F.Cu") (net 1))
 (segment (start 62.7714 33.6015) (end 62.7714 29.9219) (width 0.5) (layer "F.Cu") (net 1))
 (segment (start 66.141 30.9575) (end 66.705 30.9575) (width 0.5) (layer "F.Cu") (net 1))
 (segment (start 62.0224 38.0238) (end 46.7512 53.295) (width 0.5) (layer "F.Cu") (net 1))
 (segment (start 45.0686 38.8451) (end 44.4343 38.2108) (width 0.5) (layer "F.Cu") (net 1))
 (segment (start 31.375 47.45) (end 27.777 47.45) (width 0.5) (layer "F.Cu") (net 1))
 (segment (start 63.1342 33.9643) (end 62.7714 33.6015) (width 0.5) (layer "F.Cu") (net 1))
 (segment (start 68.6778 30.9575) (end 68.6778 35.9524) (width 0.5) (layer "F.Cu") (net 1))
 (segment (start 43.933 48.2885) (end 45.0686 47.1529) (width 0.5) (layer "F.Cu") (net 1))
 (segment (start 66.705 30.9575) (end 68.6778 30.9575) (width 0.5) (layer "F.Cu") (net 1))
 (segment (start 21.6605 54.8) (end 21.6605 50.7322) (width 0.5) (layer "F.Cu") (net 1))
 (segment (start 21.6605 50.7322) (end 20.1594 49.2311) (width 0.5) (layer "F.Cu") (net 1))
 (segment (start 24.4948 50.7322) (end 21.6605 50.7322) (width 0.5) (layer "F.Cu") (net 1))
 (segment (start 66.705 30.9575) (end 66.705 30) (width 0.5) (layer "F.Cu") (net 1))
 (segment (start 72.73 30) (end 71.4283 30) (width 0.5) (layer "F.Cu") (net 1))
 (segment (start 16.9059 47.6925) (end 17.8059 48.5925) (width 0.5) (layer "F.Cu") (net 1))
 (segment (start 70.4708 30.9575) (end 71.4283 30) (width 0.5) (layer "F.Cu") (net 1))
 (segment (start 40.8523 49.1057) (end 40.0493 49.9087) (width 0.25) (layer "F.Cu") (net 8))
 (segment (start 38.8512 42.6921) (end 38.7512 42.5921) (width 0.25) (layer "F.Cu") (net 8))
 (segment (start 38.8512 42.6921) (end 40.8523 44.6932) (width 0.25) (layer "F.Cu") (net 8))
 (segment (start 38.7512 42.5921) (end 38.7512 40.7721) (width 0.25) (layer "F.Cu") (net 8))
 (segment (start 40.8523 44.6932) (end 40.8523 49.1057) (width 0.25) (layer "F.Cu") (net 8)))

